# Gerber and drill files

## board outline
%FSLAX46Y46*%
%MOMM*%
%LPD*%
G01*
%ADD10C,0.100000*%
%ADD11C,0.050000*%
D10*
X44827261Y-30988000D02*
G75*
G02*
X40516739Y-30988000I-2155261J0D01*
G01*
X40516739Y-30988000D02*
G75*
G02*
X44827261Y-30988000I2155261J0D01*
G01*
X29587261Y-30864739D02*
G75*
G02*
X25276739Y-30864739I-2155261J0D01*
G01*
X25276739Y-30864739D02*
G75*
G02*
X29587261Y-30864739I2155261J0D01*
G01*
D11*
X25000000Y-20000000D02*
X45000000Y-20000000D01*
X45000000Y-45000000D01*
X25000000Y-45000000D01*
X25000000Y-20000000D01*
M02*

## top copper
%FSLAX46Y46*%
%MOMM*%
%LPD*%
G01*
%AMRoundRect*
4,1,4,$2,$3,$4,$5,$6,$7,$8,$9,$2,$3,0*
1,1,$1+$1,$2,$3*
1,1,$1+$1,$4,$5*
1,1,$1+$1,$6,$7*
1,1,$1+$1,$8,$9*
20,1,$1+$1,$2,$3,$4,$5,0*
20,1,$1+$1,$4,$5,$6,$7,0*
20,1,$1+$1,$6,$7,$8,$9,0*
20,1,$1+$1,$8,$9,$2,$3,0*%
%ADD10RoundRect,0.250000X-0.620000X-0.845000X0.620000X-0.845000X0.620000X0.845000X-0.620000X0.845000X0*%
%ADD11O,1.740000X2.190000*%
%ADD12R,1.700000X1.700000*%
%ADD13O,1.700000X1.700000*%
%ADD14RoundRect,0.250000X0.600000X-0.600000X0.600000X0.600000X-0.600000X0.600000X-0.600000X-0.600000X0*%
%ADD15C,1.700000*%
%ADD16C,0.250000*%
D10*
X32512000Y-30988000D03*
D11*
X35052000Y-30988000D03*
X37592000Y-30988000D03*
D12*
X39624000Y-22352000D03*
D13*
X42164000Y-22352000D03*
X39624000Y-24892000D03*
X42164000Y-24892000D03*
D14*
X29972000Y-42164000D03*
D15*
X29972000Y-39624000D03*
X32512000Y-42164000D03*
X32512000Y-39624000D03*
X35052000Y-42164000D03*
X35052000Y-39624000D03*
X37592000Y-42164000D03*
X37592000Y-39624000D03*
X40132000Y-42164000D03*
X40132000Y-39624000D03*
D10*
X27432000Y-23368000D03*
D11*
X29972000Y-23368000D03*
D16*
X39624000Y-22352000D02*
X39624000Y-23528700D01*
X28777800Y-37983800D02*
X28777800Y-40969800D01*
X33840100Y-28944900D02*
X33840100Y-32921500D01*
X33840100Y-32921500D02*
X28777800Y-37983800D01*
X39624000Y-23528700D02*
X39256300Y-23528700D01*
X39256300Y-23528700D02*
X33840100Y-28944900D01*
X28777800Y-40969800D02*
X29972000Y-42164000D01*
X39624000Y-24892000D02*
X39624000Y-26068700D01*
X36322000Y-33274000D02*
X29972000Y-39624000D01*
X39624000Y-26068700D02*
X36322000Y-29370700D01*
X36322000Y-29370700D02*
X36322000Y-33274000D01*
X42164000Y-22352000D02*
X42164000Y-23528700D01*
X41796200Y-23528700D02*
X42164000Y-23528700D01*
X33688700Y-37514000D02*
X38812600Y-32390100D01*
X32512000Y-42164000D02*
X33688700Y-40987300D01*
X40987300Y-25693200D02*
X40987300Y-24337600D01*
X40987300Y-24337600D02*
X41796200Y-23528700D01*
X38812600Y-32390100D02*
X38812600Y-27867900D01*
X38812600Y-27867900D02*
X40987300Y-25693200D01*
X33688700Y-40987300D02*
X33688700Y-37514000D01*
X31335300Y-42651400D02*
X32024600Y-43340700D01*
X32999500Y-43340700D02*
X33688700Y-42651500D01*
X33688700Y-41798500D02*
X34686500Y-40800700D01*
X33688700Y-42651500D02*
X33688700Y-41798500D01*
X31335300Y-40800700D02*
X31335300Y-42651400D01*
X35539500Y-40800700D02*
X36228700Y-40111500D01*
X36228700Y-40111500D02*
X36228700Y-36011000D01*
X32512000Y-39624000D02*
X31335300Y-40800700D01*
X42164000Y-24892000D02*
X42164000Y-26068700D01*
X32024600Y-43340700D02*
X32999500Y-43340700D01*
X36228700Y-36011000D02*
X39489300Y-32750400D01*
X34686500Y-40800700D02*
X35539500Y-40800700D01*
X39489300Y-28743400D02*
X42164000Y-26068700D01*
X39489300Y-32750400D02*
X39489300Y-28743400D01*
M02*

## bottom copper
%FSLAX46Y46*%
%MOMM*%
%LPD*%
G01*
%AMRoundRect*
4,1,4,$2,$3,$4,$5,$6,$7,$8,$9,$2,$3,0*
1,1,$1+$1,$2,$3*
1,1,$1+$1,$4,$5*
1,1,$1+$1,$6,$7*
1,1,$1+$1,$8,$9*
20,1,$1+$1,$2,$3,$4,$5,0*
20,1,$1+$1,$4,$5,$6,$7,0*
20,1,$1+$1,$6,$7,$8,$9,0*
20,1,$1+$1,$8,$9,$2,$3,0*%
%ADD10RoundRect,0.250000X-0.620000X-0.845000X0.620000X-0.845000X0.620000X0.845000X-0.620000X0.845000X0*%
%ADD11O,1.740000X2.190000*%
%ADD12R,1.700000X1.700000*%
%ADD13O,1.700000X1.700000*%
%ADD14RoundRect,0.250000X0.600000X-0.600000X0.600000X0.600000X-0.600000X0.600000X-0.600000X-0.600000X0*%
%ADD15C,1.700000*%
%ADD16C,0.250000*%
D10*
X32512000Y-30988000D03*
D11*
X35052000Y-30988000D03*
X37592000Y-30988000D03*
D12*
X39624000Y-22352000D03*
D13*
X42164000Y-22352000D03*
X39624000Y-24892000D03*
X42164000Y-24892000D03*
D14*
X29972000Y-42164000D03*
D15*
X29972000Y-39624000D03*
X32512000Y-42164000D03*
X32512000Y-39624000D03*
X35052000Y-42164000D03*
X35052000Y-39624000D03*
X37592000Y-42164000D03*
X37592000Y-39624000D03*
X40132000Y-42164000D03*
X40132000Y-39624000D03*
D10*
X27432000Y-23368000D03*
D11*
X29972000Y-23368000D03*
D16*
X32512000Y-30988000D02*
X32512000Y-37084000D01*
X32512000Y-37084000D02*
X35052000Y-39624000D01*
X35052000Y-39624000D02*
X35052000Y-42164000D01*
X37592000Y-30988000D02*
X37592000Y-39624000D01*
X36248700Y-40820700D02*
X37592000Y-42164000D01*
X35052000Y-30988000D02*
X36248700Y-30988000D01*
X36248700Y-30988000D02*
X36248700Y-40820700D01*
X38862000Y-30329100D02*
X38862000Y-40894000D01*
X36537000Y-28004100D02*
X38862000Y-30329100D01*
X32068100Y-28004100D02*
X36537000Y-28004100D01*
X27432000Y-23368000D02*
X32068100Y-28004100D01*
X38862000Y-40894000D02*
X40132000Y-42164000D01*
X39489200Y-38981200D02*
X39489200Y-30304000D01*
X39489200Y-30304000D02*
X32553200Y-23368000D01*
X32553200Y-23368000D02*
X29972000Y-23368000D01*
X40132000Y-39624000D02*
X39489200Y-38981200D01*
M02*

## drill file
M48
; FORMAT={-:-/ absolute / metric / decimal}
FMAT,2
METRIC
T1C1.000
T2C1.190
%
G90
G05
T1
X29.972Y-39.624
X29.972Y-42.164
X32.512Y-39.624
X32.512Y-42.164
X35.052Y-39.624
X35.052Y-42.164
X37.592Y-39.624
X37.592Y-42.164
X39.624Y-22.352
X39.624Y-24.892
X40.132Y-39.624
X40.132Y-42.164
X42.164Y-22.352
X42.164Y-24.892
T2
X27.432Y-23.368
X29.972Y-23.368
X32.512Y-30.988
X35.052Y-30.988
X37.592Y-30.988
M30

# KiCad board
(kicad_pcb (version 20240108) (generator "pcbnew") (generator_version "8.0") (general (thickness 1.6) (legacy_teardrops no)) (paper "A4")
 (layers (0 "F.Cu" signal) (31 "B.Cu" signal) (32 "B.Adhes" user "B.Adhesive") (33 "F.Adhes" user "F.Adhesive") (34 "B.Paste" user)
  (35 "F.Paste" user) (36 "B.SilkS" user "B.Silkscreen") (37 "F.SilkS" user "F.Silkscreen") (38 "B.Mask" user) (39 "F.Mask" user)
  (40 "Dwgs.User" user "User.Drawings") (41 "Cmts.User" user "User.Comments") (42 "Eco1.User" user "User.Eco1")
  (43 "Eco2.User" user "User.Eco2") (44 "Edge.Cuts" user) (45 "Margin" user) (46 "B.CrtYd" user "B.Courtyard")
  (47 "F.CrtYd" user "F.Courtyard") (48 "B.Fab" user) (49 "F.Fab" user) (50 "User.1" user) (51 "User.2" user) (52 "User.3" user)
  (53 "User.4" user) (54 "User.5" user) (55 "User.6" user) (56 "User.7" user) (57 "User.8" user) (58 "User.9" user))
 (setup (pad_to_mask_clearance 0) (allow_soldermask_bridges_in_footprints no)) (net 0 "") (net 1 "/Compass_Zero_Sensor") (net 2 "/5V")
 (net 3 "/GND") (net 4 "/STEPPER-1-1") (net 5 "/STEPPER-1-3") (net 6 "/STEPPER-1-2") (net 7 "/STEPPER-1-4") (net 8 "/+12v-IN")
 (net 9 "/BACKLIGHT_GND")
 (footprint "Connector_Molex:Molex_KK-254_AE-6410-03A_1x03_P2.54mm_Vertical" (layer "F.Cu") (at 32.512 30.988)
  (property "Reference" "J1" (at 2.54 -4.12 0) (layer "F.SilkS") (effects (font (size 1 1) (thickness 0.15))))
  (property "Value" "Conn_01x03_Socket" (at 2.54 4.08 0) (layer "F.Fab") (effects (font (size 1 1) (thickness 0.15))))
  (pad "1" thru_hole roundrect (at 0 0) (size 1.74 2.19) (drill 1.19) (layers "*.Cu" "*.Mask") (remove_unused_layers no)
   (roundrect_rratio 0.143678) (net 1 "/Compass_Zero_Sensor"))
  (pad "2" thru_hole oval (at 2.54 0) (size 1.74 2.19) (drill 1.19) (layers "*.Cu" "*.Mask") (remove_unused_layers no) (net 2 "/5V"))
  (pad "3" thru_hole oval (at 5.08 0) (size 1.74 2.19) (drill 1.19) (layers "*.Cu" "*.Mask") (remove_unused_layers no) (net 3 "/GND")))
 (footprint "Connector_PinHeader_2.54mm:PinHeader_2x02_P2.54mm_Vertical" (layer "F.Cu") (at 39.624 22.352)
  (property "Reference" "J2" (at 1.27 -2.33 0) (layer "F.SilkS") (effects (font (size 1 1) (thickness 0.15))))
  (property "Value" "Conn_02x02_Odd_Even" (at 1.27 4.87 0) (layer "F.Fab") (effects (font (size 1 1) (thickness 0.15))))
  (pad "1" thru_hole rect (at 0 0) (size 1.7 1.7) (drill 1) (layers "*.Cu" "*.Mask") (remove_unused_layers no) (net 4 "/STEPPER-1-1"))
  (pad "2" thru_hole oval (at 2.54 0) (size 1.7 1.7) (drill 1) (layers "*.Cu" "*.Mask") (remove_unused_layers no) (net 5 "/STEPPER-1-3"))
  (pad "3" thru_hole oval (at 0 2.54) (size 1.7 1.7) (drill 1) (layers "*.Cu" "*.Mask") (remove_unused_layers no) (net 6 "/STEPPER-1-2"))
  (pad "4" thru_hole oval (at 2.54 2.54) (size 1.7 1.7) (drill 1) (layers "*.Cu" "*.Mask") (remove_unused_layers no) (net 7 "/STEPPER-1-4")))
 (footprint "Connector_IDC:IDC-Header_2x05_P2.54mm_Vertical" (layer "F.Cu") (at 29.972 42.164 90)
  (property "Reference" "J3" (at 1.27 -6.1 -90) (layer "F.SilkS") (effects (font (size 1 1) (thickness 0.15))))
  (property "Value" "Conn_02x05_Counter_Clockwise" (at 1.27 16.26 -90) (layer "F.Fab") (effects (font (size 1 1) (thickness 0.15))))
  (pad "1" thru_hole roundrect (at 0 0 90) (size 1.7 1.7) (drill 1) (layers "*.Cu" "*.Mask") (remove_unused_layers no)
   (roundrect_rratio 0.147059) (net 4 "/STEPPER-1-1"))
  (pad "2" thru_hole circle (at 2.54 0 90) (size 1.7 1.7) (drill 1) (layers "*.Cu" "*.Mask") (remove_unused_layers no)
   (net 6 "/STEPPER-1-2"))
  (pad "3" thru_hole circle (at 0 2.54 90) (size 1.7 1.7) (drill 1) (layers "*.Cu" "*.Mask") (remove_unused_layers no)
   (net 5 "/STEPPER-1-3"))
  (pad "4" thru_hole circle (at 2.54 2.54 90) (size 1.7 1.7) (drill 1) (layers "*.Cu" "*.Mask") (remove_unused_layers no)
   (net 7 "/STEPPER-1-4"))
  (pad "5" thru_hole circle (at 0 5.08 90) (size 1.7 1.7) (drill 1) (layers "*.Cu" "*.Mask") (remove_unused_layers no)
   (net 1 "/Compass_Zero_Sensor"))
  (pad "6" thru_hole circle (at 2.54 5.08 90) (size 1.7 1.7) (drill 1) (layers "*.Cu" "*.Mask") (remove_unused_layers no)
   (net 1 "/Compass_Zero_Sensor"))
  (pad "7" thru_hole circle (at 0 7.62 90) (size 1.7 1.7) (drill 1) (layers "*.Cu" "*.Mask") (remove_unused_layers no) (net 2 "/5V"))
  (pad "8" thru_hole circle (at 2.54 7.62 90) (size 1.7 1.7) (drill 1) (layers "*.Cu" "*.Mask") (remove_unused_layers no) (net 3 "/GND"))
  (pad "9" thru_hole circle (at 0 10.16 90) (size 1.7 1.7) (drill 1) (layers "*.Cu" "*.Mask") (remove_unused_layers no) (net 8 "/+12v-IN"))
  (pad "10" thru_hole circle (at 2.54 10.16 90) (size 1.7 1.7) (drill 1) (layers "*.Cu" "*.Mask") (remove_unused_layers no)
   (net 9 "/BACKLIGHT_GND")))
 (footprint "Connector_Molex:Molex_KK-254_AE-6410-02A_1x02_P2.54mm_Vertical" (layer "F.Cu") (at 27.432 23.368)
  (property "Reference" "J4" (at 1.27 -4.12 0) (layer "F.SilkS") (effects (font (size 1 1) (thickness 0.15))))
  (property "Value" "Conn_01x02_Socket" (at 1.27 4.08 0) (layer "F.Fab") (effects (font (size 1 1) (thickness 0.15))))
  (pad "1" thru_hole roundrect (at 0 0) (size 1.74 2.19) (drill 1.19) (layers "*.Cu" "*.Mask") (remove_unused_layers no)
   (roundrect_rratio 0.143678) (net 8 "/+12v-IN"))
  (pad "2" thru_hole oval (at 2.54 0) (size 1.74 2.19) (drill 1.19) (layers "*.Cu" "*.Mask") (remove_unused_layers no)
   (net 9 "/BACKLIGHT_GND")))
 (gr_circle (center 42.672 30.988) (end 44.196 32.512) (stroke (width 0.1) (type default)) (fill none) (layer "Edge.Cuts"))
 (gr_circle (center 27.432 30.864739) (end 28.956 32.388739) (stroke (width 0.1) (type default)) (fill none) (layer "Edge.Cuts"))
 (gr_rect (start 25 20) (end 45 45) (stroke (width 0.05) (type default)) (fill none) (layer "Edge.Cuts"))
 (segment (start 39.624 22.352) (end 39.624 23.5287) (width 0.25) (layer "F.Cu") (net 4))
 (segment (start 28.7778 37.9838) (end 28.7778 40.9698) (width 0.25) (layer "F.Cu") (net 4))
 (segment (start 33.8401 28.9449) (end 33.8401 32.9215) (width 0.25) (layer "F.Cu") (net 4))
 (segment (start 33.8401 32.9215) (end 28.7778 37.9838) (width 0.25) (layer "F.Cu") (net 4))
 (segment (start 39.624 23.5287) (end 39.2563 23.5287) (width 0.25) (layer "F.Cu") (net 4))
 (segment (start 39.2563 23.5287) (end 33.8401 28.9449) (width 0.25) (layer "F.Cu") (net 4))
 (segment (start 28.7778 40.9698) (end 29.972 42.164) (width 0.25) (layer "F.Cu") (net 4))
 (segment (start 39.624 24.892) (end 39.624 26.0687) (width 0.25) (layer "F.Cu") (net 6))
 (segment (start 36.322 33.274) (end 29.972 39.624) (width 0.25) (layer "F.Cu") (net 6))
 (segment (start 39.624 26.0687) (end 36.322 29.3707) (width 0.25) (layer "F.Cu") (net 6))
 (segment (start 36.322 29.3707) (end 36.322 33.274) (width 0.25) (layer "F.Cu") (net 6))
 (segment (start 42.164 22.352) (end 42.164 23.5287) (width 0.25) (layer "F.Cu") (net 5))
 (segment (start 41.7962 23.5287) (end 42.164 23.5287) (width 0.25) (layer "F.Cu") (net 5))
 (segment (start 33.6887 37.514) (end 38.8126 32.3901) (width 0.25) (layer "F.Cu") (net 5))
 (segment (start 32.512 42.164) (end 33.6887 40.9873) (width 0.25) (layer "F.Cu") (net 5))
 (segment (start 40.9873 25.6932) (end 40.9873 24.3376) (width 0.25) (layer "F.Cu") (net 5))
 (segment (start 40.9873 24.3376) (end 41.7962 23.5287) (width 0.25) (layer "F.Cu") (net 5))
 (segment (start 38.8126 32.3901) (end 38.8126 27.8679) (width 0.25) (layer "F.Cu") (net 5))
 (segment (start 38.8126 27.8679) (end 40.9873 25.6932) (width 0.25) (layer "F.Cu") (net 5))
 (segment (start 33.6887 40.9873) (end 33.6887 37.514) (width 0.25) (layer "F.Cu") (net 5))
 (segment (start 31.3353 42.6514) (end 32.0246 43.3407) (width 0.25) (layer "F.Cu") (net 7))
 (segment (start 32.9995 43.3407) (end 33.6887 42.6515) (width 0.25) (layer "F.Cu") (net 7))
 (segment (start 33.6887 41.7985) (end 34.6865 40.8007) (width 0.25) (layer "F.Cu") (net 7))
 (segment (start 33.6887 42.6515) (end 33.6887 41.7985) (width 0.25) (layer "F.Cu") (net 7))
 (segment (start 31.3353 40.8007) (end 31.3353 42.6514) (width 0.25) (layer "F.Cu") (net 7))
 (segment (start 35.5395 40.8007) (end 36.2287 40.1115) (width 0.25) (layer "F.Cu") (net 7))
 (segment (start 36.2287 40.1115) (end 36.2287 36.011) (width 0.25) (layer "F.Cu") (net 7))
 (segment (start 32.512 39.624) (end 31.3353 40.8007) (width 0.25) (layer "F.Cu") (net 7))
 (segment (start 42.164 24.892) (end 42.164 26.0687) (width 0.25) (layer "F.Cu") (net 7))
 (segment (start 32.0246 43.3407) (end 32.9995 43.3407) (width 0.25) (layer "F.Cu") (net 7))
 (segment (start 36.2287 36.011) (end 39.4893 32.7504) (width 0.25) (layer "F.Cu") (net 7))
 (segment (start 34.6865 40.8007) (end 35.5395 40.8007) (width 0.25) (layer "F.Cu") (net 7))
 (segment (start 39.4893 28.7434) (end 42.164 26.0687) (width 0.25) (layer "F.Cu") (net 7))
 (segment (start 39.4893 32.7504) (end 39.4893 28.7434) (width 0.25) (layer "F.Cu") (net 7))
 (segment (start 32.512 30.988) (end 32.512 37.084) (width 0.25) (layer "B.Cu") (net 1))
 (segment (start 32.512 37.084) (end 35.052 39.624) (width 0.25) (layer "B.Cu") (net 1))
 (segment (start 35.052 39.624) (end 35.052 42.164) (width 0.25) (layer "B.Cu") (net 1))
 (segment (start 37.592 30.988) (end 37.592 39.624) (width 0.25) (layer "B.Cu") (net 3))
 (segment (start 36.2487 40.8207) (end 37.592 42.164) (width 0.25) (layer "B.Cu") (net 2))
 (segment (start 35.052 30.988) (end 36.2487 30.988) (width 0.25) (layer "B.Cu") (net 2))
 (segment (start 36.2487 30.988) (end 36.2487 40.8207) (width 0.25) (layer "B.Cu") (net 2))
 (segment (start 38.862 30.3291) (end 38.862 40.894) (width 0.25) (layer "B.Cu") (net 8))
 (segment (start 36.537 28.0041) (end 38.862 30.3291) (width 0.25) (layer "B.Cu") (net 8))
 (segment (start 32.0681 28.0041) (end 36.537 28.0041) (width 0.25) (layer "B.Cu") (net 8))
 (segment (start 27.432 23.368) (end 32.0681 28.0041) (width 0.25) (layer "B.Cu") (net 8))
 (segment (start 38.862 40.894) (end 40.132 42.164) (width 0.25) (layer "B.Cu") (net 8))
 (segment (start 39.4892 38.9812) (end 39.4892 30.304) (width 0.25) (layer "B.Cu") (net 9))
 (segment (start 39.4892 30.304) (end 32.5532 23.368) (width 0.25) (layer "B.Cu") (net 9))
 (segment (start 32.5532 23.368) (end 29.972 23.368) (width 0.25) (layer "B.Cu") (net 9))
 (segment (start 40.132 39.624) (end 39.4892 38.9812) (width 0.25) (layer "B.Cu") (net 9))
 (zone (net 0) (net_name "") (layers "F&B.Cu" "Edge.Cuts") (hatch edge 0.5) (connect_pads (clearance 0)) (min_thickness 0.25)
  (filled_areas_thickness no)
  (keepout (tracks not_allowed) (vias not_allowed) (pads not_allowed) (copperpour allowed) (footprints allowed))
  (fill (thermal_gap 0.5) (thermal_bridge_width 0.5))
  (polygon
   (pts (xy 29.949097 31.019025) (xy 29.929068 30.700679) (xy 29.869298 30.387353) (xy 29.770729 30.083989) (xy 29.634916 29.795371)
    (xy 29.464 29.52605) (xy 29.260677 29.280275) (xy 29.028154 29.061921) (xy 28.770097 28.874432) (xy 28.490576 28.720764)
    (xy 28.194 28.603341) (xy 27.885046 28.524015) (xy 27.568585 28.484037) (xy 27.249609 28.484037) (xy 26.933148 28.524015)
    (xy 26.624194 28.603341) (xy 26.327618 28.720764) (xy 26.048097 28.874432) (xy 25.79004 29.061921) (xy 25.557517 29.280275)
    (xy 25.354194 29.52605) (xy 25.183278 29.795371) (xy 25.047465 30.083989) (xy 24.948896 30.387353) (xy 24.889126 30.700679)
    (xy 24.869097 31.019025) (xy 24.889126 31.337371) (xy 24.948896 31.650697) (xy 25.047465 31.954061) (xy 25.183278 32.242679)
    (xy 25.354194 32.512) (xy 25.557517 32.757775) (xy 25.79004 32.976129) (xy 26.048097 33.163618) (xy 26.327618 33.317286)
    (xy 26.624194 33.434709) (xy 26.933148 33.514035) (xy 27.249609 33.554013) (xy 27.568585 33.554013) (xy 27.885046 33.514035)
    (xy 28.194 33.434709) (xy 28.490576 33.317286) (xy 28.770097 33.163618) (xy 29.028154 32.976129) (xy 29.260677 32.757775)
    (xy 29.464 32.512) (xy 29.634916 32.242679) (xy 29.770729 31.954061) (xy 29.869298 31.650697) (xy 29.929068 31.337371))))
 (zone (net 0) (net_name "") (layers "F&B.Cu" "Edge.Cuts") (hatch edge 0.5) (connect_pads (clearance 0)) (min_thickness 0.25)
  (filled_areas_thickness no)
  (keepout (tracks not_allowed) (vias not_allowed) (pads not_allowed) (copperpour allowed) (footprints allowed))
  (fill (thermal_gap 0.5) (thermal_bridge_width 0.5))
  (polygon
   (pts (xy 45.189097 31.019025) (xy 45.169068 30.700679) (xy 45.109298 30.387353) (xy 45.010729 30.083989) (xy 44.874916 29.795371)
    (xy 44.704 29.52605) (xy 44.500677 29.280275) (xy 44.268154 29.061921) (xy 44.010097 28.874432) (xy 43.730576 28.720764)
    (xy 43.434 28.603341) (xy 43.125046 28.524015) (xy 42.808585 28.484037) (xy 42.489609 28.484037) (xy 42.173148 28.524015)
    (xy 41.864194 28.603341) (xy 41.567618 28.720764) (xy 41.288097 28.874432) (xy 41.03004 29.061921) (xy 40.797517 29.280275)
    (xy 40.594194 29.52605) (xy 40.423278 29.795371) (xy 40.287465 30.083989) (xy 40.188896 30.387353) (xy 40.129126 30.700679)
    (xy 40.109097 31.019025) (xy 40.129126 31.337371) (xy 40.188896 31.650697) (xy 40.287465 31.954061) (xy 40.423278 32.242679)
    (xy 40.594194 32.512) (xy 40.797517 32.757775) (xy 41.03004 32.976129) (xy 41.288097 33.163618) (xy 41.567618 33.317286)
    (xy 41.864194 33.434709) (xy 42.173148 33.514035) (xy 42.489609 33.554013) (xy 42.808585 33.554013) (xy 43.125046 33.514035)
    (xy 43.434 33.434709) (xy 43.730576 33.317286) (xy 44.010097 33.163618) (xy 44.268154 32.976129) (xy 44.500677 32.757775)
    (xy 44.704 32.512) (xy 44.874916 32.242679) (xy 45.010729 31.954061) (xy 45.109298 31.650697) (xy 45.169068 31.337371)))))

